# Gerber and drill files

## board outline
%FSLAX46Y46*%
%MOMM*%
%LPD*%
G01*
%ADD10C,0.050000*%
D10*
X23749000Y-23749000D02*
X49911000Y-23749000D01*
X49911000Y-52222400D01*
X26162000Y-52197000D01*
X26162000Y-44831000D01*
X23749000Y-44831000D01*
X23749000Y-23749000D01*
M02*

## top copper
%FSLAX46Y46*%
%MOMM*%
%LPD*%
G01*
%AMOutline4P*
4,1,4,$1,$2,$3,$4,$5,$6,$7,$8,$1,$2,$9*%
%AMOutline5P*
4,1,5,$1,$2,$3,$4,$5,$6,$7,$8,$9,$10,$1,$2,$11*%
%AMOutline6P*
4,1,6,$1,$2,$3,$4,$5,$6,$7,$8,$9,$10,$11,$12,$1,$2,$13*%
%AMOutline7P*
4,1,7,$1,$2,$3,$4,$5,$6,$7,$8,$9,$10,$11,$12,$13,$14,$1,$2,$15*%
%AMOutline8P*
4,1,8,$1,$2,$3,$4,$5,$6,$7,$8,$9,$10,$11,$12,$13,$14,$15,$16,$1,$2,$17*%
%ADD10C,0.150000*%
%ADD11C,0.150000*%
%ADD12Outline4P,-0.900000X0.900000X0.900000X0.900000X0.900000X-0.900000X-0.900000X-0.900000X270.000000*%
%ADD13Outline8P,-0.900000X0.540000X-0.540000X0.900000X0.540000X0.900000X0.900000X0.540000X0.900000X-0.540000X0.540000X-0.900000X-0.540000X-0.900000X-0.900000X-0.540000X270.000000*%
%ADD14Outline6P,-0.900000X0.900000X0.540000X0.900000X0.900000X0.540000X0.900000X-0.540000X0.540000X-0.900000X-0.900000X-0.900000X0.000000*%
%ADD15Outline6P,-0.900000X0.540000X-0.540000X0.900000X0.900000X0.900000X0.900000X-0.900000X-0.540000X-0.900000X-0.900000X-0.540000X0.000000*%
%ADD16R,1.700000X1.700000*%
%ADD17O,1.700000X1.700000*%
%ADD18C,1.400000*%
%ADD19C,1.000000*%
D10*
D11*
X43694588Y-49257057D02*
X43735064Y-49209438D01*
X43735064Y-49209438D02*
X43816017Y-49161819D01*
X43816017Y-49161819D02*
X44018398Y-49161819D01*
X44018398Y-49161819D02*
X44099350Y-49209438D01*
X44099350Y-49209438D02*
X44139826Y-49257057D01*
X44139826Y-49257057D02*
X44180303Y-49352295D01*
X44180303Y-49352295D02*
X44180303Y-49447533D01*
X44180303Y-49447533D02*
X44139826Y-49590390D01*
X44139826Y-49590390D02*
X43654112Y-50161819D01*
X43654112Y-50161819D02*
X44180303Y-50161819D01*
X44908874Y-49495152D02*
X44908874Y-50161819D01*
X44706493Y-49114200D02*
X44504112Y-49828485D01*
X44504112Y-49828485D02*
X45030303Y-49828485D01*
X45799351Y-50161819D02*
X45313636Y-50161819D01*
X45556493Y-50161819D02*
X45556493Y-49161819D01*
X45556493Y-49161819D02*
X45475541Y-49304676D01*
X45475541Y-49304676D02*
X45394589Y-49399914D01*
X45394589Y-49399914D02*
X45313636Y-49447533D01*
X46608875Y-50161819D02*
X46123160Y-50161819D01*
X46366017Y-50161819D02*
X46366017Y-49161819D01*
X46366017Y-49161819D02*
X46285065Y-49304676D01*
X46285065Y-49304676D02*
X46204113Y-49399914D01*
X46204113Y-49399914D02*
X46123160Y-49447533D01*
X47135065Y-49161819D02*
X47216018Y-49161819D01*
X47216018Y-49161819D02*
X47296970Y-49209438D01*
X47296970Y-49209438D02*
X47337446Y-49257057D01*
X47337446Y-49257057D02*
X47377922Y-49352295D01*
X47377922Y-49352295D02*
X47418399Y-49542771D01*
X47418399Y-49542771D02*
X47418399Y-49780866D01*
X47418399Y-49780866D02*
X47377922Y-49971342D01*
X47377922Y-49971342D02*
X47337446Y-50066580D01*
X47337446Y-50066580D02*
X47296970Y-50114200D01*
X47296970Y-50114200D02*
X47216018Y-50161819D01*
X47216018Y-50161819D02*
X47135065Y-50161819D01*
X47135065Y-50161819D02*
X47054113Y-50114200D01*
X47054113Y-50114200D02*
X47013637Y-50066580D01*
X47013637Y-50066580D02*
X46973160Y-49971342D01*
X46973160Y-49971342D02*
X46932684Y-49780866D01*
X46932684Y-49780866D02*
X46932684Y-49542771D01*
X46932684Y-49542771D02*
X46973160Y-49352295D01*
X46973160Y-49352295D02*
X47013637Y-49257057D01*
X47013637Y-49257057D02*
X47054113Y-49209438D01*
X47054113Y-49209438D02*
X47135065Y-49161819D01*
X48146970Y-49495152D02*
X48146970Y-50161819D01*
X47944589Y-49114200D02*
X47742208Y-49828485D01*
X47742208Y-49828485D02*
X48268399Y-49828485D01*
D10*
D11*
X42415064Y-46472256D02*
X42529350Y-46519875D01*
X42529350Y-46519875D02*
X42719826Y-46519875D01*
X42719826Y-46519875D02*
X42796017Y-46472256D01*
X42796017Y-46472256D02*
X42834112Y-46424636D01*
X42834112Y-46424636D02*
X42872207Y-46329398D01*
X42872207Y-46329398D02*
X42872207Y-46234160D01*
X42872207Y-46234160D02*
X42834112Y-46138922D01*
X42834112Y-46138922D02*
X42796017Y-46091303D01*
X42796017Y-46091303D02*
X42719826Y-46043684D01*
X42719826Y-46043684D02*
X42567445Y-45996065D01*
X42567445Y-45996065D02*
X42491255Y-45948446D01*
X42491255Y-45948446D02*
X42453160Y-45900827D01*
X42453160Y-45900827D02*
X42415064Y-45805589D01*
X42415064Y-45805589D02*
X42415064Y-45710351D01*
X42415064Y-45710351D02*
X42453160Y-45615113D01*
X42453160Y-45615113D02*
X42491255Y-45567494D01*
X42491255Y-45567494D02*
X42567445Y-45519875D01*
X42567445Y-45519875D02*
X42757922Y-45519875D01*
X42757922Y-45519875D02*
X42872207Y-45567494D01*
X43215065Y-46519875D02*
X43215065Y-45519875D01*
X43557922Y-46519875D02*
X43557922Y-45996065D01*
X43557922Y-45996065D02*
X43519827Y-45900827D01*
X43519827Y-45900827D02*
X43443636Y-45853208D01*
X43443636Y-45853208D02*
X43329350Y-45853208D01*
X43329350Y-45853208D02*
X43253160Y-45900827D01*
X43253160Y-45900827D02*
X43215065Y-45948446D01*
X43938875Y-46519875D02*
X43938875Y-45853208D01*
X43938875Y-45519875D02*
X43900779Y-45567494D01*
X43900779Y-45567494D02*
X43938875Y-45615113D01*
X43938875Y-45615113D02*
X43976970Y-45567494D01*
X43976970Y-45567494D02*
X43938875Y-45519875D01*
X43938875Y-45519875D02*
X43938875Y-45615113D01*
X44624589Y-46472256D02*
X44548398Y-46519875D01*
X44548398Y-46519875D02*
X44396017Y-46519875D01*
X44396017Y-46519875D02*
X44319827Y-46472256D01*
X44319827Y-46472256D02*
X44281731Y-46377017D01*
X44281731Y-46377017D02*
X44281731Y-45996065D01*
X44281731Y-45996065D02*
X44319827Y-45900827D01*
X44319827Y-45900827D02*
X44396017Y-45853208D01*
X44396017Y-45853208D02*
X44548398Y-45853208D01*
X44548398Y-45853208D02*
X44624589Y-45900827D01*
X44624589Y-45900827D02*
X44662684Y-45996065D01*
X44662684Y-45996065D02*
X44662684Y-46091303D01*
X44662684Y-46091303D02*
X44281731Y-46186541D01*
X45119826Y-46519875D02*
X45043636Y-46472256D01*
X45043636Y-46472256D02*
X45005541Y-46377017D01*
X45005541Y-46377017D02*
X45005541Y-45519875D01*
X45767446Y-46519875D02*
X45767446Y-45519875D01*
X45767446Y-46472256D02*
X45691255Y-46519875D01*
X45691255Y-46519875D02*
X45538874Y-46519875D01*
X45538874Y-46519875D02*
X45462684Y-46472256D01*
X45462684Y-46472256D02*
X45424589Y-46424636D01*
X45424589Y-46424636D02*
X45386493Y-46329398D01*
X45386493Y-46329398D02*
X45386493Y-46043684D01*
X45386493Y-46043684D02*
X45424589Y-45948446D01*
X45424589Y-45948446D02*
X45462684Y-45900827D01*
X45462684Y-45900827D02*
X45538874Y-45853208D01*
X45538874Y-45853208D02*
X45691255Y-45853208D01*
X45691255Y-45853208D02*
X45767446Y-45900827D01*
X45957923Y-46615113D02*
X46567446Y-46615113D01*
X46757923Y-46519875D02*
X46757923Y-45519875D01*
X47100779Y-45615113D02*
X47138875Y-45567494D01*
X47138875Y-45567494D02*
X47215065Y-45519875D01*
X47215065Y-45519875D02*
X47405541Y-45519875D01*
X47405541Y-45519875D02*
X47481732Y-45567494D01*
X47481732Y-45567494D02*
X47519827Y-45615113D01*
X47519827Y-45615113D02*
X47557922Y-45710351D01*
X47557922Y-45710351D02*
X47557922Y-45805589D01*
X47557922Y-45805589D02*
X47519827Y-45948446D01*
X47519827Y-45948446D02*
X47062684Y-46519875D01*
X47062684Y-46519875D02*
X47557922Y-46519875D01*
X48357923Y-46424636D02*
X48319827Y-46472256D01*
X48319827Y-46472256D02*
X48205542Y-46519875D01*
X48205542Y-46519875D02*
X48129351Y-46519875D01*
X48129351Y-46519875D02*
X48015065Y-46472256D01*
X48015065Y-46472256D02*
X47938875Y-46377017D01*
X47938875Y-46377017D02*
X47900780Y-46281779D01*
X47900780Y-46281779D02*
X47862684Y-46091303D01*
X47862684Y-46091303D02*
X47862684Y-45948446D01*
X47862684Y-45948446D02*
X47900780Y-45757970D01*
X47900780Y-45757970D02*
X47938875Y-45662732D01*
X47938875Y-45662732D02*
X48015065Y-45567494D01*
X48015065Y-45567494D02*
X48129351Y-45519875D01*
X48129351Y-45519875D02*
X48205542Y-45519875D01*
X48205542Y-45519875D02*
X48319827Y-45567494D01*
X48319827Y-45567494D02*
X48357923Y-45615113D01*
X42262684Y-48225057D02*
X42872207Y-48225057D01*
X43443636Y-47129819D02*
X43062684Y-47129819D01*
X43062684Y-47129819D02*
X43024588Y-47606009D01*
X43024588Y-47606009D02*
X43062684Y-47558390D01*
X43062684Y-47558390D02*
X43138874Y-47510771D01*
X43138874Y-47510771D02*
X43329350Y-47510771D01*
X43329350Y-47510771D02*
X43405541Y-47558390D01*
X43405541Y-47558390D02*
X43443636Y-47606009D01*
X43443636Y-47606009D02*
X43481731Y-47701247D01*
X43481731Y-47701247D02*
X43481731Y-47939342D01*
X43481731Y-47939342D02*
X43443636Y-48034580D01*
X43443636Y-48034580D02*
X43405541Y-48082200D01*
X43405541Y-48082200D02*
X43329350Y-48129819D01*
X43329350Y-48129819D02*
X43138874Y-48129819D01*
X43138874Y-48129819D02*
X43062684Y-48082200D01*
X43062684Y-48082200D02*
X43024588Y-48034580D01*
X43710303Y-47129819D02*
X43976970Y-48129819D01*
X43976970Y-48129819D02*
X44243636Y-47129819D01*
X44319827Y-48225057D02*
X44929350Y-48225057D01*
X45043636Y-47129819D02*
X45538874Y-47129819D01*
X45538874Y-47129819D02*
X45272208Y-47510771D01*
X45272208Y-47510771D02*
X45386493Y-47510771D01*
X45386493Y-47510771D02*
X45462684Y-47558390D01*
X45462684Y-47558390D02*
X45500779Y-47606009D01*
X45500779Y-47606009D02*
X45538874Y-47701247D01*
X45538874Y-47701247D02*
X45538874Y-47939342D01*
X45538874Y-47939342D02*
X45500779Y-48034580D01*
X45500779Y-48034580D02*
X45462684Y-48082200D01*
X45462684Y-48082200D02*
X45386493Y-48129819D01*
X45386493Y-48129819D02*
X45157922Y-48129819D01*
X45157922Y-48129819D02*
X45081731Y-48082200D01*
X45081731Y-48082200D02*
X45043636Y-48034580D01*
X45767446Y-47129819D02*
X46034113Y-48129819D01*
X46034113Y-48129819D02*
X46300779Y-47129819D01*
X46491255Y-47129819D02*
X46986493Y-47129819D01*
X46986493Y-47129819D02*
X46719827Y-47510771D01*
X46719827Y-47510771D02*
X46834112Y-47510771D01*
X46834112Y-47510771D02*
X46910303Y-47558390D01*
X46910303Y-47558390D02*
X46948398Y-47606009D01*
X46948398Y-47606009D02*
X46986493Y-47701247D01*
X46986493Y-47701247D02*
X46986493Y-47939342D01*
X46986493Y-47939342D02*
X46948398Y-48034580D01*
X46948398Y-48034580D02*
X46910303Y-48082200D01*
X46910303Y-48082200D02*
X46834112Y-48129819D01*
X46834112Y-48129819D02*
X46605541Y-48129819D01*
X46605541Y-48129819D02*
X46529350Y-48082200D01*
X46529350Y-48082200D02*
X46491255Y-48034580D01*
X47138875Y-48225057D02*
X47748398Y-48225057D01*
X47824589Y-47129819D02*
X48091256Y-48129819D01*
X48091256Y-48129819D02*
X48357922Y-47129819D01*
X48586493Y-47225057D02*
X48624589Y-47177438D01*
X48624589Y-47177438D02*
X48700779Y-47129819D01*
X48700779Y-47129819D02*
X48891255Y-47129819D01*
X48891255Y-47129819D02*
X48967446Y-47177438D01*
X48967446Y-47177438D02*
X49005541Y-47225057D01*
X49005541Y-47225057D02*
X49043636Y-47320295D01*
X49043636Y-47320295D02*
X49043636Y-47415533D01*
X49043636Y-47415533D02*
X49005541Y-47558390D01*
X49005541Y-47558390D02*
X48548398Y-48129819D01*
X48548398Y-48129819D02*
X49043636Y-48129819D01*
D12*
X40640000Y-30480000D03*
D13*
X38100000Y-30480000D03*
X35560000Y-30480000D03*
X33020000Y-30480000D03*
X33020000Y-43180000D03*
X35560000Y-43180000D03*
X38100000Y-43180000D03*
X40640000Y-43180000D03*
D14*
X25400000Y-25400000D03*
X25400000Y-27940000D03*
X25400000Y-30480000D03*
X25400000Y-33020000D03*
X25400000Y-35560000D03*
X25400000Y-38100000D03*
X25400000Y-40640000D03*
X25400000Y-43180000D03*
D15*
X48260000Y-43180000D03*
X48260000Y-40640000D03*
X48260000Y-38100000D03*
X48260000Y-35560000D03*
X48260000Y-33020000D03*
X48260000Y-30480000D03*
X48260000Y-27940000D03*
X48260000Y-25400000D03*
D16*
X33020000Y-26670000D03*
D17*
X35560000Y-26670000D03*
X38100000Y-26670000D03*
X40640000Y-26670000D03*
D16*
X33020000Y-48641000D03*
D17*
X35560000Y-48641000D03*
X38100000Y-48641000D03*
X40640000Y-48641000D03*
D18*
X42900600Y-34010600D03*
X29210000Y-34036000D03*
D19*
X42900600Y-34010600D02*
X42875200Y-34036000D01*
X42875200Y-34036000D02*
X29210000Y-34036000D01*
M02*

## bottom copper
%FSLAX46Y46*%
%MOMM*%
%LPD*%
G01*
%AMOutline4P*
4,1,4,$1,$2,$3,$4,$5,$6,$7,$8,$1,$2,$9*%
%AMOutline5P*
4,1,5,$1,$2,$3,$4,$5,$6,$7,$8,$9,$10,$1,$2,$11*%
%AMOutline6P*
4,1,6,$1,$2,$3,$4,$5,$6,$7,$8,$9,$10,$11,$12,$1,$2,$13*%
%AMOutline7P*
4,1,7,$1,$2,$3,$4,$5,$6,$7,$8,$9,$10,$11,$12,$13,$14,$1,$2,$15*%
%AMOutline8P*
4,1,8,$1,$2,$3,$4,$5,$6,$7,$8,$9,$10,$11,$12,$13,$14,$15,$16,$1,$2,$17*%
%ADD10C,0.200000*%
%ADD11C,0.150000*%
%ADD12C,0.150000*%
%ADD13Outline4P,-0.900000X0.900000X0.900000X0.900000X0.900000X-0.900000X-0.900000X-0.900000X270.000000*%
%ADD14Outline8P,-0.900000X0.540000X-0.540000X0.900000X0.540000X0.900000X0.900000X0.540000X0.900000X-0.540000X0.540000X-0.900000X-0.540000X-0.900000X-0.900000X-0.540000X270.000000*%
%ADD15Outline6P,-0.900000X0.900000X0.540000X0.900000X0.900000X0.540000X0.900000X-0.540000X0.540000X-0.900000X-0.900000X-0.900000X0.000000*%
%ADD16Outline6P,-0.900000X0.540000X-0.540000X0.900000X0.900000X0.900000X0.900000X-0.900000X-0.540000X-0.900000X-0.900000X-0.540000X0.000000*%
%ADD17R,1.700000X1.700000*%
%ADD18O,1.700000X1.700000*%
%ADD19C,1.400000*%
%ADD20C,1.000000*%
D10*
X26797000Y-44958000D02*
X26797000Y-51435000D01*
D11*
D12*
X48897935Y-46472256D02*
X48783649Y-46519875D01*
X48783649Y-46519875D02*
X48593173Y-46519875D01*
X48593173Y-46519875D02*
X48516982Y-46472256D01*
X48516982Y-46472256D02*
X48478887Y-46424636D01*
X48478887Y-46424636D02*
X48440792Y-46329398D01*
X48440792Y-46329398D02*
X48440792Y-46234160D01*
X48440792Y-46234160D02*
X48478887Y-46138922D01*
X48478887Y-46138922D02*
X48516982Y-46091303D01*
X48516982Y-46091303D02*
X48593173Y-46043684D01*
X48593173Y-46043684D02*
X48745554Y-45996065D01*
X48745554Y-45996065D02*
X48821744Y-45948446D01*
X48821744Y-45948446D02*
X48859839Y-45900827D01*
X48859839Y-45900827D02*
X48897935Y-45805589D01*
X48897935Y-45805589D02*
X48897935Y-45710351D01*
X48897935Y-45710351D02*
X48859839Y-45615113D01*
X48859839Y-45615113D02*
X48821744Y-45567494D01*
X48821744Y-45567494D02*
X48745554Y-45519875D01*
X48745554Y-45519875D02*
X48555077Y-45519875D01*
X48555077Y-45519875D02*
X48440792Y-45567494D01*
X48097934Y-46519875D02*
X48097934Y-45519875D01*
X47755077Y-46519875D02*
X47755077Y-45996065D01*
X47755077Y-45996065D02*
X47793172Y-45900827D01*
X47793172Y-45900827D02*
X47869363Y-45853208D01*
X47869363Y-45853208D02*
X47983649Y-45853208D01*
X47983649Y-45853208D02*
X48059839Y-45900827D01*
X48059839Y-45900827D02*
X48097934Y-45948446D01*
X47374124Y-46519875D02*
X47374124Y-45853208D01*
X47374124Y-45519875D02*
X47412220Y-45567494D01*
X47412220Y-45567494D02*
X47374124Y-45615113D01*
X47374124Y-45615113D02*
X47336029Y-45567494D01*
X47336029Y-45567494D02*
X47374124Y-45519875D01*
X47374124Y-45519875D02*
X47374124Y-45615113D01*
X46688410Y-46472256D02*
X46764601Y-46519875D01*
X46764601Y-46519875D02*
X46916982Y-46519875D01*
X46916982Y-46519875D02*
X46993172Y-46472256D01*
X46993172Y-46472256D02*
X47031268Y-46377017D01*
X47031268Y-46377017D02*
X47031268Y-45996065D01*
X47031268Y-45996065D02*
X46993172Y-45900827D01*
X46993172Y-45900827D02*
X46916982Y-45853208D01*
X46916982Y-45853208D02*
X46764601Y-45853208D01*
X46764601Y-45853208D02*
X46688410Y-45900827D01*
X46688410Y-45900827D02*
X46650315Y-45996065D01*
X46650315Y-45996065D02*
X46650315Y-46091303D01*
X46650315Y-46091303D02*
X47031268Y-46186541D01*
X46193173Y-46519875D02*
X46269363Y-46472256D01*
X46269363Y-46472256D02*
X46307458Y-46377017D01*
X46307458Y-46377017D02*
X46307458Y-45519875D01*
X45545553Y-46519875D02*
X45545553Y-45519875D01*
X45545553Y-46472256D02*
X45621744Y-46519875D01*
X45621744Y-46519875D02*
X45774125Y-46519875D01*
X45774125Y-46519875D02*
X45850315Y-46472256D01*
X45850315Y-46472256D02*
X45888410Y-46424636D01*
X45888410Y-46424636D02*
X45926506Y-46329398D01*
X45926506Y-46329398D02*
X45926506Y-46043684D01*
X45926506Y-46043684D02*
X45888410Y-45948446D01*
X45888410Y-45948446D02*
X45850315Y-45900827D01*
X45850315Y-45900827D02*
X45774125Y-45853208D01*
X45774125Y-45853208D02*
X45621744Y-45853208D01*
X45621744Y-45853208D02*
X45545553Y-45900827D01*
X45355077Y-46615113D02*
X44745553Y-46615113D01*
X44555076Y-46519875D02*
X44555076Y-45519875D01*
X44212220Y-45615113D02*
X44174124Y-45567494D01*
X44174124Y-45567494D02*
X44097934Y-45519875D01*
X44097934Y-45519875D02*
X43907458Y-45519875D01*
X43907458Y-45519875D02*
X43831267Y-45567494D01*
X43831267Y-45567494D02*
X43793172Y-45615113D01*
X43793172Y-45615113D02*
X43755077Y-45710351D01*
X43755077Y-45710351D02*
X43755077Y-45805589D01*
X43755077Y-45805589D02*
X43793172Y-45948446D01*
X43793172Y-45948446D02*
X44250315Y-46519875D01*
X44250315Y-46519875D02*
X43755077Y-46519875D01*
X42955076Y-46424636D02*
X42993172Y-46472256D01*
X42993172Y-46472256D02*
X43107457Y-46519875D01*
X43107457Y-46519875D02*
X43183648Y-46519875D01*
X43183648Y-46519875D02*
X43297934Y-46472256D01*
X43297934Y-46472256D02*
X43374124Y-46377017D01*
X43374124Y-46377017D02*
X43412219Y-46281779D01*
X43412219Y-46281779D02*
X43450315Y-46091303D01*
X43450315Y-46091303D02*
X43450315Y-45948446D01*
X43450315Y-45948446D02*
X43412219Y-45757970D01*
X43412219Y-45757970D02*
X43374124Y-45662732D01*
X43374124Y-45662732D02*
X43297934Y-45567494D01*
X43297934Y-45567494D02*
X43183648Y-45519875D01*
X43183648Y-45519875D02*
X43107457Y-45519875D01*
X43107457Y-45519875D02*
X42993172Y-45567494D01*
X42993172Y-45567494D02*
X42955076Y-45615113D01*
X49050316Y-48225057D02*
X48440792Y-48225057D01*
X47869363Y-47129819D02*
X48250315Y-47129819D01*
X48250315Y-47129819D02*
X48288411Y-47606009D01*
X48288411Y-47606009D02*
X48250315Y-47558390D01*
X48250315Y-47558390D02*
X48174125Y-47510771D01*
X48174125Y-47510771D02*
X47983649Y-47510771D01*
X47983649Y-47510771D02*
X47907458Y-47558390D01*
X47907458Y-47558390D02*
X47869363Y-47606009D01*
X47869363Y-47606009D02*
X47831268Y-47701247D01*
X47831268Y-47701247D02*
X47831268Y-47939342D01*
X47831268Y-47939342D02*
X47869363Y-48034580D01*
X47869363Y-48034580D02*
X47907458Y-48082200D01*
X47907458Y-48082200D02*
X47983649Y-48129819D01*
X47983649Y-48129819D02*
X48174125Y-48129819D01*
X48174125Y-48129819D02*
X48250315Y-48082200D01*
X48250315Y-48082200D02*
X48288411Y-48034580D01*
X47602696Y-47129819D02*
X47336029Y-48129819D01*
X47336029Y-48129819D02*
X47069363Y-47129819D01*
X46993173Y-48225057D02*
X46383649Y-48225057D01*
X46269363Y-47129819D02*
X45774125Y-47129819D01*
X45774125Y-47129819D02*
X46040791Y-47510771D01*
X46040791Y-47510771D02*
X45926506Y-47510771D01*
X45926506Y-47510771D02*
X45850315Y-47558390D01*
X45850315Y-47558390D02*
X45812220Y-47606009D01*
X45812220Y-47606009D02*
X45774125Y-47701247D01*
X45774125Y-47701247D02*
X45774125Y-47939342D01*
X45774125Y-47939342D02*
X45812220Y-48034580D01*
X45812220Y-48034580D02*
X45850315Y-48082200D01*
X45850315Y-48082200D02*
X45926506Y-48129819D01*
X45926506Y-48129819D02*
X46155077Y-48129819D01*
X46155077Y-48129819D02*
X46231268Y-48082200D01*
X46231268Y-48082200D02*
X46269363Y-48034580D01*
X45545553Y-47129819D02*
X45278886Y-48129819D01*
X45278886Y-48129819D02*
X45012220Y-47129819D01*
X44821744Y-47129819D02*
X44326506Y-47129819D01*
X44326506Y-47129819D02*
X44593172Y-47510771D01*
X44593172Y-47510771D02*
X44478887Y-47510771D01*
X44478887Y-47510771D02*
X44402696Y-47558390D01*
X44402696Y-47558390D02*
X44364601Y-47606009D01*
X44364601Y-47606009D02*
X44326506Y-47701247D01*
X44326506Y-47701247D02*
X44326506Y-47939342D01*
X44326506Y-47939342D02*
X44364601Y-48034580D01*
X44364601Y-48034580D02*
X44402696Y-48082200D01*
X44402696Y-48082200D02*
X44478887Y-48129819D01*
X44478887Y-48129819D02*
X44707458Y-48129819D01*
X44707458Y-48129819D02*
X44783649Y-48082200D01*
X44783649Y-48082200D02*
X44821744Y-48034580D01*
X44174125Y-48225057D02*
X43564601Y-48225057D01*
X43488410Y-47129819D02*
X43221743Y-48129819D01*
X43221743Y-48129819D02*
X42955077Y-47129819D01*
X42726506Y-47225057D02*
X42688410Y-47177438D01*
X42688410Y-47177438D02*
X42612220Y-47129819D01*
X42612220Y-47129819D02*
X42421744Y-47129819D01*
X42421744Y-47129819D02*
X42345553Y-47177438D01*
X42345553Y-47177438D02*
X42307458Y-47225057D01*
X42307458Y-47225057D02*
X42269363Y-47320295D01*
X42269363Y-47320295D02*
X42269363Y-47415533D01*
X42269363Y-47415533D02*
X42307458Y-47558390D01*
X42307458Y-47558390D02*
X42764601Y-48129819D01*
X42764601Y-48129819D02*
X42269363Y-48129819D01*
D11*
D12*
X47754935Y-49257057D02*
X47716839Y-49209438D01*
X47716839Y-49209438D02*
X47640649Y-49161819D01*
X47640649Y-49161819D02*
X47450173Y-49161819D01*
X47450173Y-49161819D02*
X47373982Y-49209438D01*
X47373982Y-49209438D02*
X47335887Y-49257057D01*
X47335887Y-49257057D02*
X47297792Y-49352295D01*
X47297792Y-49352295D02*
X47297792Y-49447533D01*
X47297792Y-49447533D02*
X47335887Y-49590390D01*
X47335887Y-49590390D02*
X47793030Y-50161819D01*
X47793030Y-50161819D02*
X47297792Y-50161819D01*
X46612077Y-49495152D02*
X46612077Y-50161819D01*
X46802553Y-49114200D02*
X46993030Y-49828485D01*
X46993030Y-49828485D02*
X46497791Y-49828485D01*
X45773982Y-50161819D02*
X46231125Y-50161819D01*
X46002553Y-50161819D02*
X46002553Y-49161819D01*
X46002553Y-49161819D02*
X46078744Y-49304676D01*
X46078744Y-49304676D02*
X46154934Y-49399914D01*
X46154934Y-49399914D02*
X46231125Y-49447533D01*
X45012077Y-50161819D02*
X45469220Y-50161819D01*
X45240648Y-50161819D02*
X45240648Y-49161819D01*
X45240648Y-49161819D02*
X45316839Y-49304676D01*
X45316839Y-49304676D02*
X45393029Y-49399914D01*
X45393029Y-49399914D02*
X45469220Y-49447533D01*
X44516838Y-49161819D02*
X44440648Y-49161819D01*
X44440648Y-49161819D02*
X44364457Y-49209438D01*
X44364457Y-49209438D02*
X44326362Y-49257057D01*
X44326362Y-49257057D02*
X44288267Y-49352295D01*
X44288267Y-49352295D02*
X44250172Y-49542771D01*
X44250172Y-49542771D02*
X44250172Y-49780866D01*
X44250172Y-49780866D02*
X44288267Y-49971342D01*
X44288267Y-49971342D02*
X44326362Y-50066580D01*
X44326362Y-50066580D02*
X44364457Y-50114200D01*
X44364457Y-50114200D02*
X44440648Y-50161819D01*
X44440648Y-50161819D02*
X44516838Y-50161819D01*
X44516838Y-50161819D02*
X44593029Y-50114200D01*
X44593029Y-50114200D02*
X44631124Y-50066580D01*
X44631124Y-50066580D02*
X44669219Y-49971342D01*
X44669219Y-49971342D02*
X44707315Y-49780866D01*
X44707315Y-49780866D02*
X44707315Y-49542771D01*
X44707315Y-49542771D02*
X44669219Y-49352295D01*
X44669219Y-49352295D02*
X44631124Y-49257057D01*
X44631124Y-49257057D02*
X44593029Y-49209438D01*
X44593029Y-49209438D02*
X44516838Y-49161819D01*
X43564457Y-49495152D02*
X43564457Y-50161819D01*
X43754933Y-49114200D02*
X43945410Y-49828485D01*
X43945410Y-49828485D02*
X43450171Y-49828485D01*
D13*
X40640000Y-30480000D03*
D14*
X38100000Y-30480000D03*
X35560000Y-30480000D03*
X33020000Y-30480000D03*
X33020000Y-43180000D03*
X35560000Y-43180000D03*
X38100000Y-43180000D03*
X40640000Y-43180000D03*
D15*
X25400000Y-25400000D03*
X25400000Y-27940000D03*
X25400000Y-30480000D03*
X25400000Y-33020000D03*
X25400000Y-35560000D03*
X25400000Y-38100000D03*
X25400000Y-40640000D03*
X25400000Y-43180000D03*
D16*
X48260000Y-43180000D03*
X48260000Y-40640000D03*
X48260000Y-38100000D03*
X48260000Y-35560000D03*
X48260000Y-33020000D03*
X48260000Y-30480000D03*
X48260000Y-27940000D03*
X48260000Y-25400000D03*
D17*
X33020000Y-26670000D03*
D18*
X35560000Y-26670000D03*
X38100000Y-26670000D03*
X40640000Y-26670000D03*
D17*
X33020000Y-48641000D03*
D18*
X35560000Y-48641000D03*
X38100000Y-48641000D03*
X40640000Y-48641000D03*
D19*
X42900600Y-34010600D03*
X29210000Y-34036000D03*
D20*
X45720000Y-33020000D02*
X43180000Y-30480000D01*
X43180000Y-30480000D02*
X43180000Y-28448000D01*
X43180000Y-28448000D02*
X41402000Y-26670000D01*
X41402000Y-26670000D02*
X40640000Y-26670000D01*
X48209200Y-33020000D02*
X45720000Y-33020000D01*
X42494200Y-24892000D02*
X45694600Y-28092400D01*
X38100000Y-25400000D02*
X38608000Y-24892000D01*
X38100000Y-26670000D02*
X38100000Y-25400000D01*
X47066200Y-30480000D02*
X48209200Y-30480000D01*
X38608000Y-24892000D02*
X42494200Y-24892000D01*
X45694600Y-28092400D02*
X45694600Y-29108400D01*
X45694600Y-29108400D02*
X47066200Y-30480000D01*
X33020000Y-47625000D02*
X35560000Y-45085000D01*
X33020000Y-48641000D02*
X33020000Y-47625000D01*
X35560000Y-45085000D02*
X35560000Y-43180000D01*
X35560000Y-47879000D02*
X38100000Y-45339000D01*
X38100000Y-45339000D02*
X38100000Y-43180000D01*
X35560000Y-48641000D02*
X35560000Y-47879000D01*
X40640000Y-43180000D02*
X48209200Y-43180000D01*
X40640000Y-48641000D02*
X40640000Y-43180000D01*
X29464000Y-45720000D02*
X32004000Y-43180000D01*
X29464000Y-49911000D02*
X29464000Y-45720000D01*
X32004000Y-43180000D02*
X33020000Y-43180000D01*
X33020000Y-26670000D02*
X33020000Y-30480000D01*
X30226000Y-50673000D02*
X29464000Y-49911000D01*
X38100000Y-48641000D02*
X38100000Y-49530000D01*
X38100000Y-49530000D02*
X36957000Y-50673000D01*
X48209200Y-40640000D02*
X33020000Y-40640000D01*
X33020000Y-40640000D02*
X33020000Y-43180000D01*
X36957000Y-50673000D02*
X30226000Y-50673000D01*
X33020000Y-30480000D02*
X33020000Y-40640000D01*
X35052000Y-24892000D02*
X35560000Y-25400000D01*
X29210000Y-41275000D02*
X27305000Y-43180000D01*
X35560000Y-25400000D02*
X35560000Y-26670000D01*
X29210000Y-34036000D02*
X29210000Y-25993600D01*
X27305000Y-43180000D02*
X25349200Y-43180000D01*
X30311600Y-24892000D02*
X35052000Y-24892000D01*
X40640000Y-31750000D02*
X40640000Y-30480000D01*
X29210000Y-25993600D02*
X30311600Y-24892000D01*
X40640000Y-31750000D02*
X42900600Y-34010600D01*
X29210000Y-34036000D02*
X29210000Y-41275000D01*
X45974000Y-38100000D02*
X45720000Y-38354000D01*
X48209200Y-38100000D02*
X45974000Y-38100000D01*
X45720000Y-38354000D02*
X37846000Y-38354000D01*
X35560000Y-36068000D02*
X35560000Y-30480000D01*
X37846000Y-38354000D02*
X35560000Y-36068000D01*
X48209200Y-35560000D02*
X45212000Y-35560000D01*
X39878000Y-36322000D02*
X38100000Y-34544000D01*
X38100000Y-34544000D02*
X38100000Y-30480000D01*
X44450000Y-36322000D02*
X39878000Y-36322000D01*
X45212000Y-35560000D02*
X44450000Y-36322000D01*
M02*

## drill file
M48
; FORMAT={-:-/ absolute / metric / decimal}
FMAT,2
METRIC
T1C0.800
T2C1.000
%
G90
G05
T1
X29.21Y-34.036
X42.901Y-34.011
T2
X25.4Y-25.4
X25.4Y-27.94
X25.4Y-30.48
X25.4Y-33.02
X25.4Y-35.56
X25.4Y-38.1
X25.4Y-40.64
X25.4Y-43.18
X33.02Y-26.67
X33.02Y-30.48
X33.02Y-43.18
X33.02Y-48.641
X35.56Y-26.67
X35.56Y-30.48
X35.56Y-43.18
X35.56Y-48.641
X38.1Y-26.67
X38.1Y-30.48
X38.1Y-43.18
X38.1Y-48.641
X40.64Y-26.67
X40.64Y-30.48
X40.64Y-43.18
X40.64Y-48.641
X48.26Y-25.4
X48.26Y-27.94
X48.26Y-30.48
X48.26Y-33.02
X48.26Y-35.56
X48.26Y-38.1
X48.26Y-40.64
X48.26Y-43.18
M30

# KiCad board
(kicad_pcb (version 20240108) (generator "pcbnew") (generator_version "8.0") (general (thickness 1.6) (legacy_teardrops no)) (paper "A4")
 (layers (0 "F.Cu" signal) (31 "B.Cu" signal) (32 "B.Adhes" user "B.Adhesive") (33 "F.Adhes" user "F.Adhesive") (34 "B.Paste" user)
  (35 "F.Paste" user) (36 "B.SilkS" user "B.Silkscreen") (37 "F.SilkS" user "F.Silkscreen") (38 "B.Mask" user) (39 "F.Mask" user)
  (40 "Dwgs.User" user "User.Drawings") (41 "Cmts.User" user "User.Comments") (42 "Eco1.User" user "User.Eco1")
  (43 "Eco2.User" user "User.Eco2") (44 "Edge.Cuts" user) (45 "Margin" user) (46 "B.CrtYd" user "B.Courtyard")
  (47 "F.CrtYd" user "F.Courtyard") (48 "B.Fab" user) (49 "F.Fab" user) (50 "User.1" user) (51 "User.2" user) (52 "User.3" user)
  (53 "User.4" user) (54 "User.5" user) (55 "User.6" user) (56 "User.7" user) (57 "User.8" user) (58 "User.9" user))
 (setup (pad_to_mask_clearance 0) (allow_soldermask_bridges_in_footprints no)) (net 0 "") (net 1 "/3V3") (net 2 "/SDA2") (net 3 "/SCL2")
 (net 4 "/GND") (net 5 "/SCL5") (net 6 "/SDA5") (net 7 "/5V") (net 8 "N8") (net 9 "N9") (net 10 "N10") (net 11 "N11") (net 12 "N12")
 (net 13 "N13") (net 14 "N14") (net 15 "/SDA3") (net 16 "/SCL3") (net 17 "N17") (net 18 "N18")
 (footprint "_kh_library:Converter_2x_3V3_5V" (layer "F.Cu") (at 40.64 30.48 -90)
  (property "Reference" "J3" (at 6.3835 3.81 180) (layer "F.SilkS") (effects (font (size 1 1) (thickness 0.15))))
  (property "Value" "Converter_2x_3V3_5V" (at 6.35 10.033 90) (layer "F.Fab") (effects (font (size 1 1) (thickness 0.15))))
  (pad "1" thru_hole roundrect (at 0 0 270) (size 1.8 1.8) (drill 1) (layers "*.Cu" "*.Mask") (remove_unused_layers no) (roundrect_rratio 0)
   (chamfer_ratio 0.2) (chamfer) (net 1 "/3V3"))
  (pad "2" thru_hole roundrect (at 0 2.54 270) (size 1.8 1.8) (drill 1) (layers "*.Cu" "*.Mask") (remove_unused_layers no)
   (roundrect_rratio 0) (chamfer_ratio 0.2) (chamfer top_left top_right bottom_left bottom_right) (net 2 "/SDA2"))
  (pad "3" thru_hole roundrect (at 0 5.08 270) (size 1.8 1.8) (drill 1) (layers "*.Cu" "*.Mask") (remove_unused_layers no)
   (roundrect_rratio 0) (chamfer_ratio 0.2) (chamfer top_left top_right bottom_left bottom_right) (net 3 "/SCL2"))
  (pad "4" thru_hole roundrect (at 0 7.62 270) (size 1.8 1.8) (drill 1) (layers "*.Cu" "*.Mask") (remove_unused_layers no)
   (roundrect_rratio 0) (chamfer_ratio 0.2) (chamfer top_left top_right bottom_left bottom_right) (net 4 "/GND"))
  (pad "5" thru_hole roundrect (at 12.7 7.62 270) (size 1.8 1.8) (drill 1) (layers "*.Cu" "*.Mask") (remove_unused_layers no)
   (roundrect_rratio 0) (chamfer_ratio 0.2) (chamfer top_left top_right bottom_left bottom_right) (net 4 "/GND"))
  (pad "6" thru_hole roundrect (at 12.7 5.08 270) (size 1.8 1.8) (drill 1) (layers "*.Cu" "*.Mask") (remove_unused_layers no)
   (roundrect_rratio 0) (chamfer_ratio 0.2) (chamfer top_left top_right bottom_left bottom_right) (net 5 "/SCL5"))
  (pad "7" thru_hole roundrect (at 12.7 2.54 270) (size 1.8 1.8) (drill 1) (layers "*.Cu" "*.Mask") (remove_unused_layers no)
   (roundrect_rratio 0) (chamfer_ratio 0.2) (chamfer top_left top_right bottom_left bottom_right) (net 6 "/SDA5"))
  (pad "8" thru_hole roundrect (at 12.7 0 270) (size 1.8 1.8) (drill 1) (layers "*.Cu" "*.Mask") (remove_unused_layers no)
   (roundrect_rratio 0) (chamfer_ratio 0.2) (chamfer top_left top_right bottom_left bottom_right) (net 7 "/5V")))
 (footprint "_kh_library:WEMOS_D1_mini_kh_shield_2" (layer "F.Cu") (at 25.4 25.4)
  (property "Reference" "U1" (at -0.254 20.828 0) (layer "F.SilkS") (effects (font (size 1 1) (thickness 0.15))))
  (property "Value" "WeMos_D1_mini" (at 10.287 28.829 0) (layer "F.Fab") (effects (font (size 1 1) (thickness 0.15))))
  (pad "1" thru_hole roundrect (at 0 0) (size 1.8 1.8) (drill 1) (layers "*.Cu" "*.Mask") (remove_unused_layers no) (roundrect_rratio 0)
   (chamfer_ratio 0.2) (chamfer top_right bottom_right) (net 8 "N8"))
  (pad "2" thru_hole roundrect (at 0 2.54) (size 1.8 1.8) (drill 1) (layers "*.Cu" "*.Mask") (remove_unused_layers no) (roundrect_rratio 0)
   (chamfer_ratio 0.2) (chamfer top_right bottom_right) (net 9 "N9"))
  (pad "3" thru_hole roundrect (at 0 5.08) (size 1.8 1.8) (drill 1) (layers "*.Cu" "*.Mask") (remove_unused_layers no) (roundrect_rratio 0)
   (chamfer_ratio 0.2) (chamfer top_right bottom_right) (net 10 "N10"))
  (pad "4" thru_hole roundrect (at 0 7.62) (size 1.8 1.8) (drill 1) (layers "*.Cu" "*.Mask") (remove_unused_layers no) (roundrect_rratio 0)
   (chamfer_ratio 0.2) (chamfer top_right bottom_right) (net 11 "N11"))
  (pad "5" thru_hole roundrect (at 0 10.16) (size 1.8 1.8) (drill 1) (layers "*.Cu" "*.Mask") (remove_unused_layers no) (roundrect_rratio 0)
   (chamfer_ratio 0.2) (chamfer top_right bottom_right) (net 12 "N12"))
  (pad "6" thru_hole roundrect (at 0 12.7) (size 1.8 1.8) (drill 1) (layers "*.Cu" "*.Mask") (remove_unused_layers no) (roundrect_rratio 0)
   (chamfer_ratio 0.2) (chamfer top_right bottom_right) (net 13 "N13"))
  (pad "7" thru_hole roundrect (at 0 15.24) (size 1.8 1.8) (drill 1) (layers "*.Cu" "*.Mask") (remove_unused_layers no) (roundrect_rratio 0)
   (chamfer_ratio 0.2) (chamfer top_right bottom_right) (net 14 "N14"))
  (pad "8" thru_hole roundrect (at 0 17.78) (size 1.8 1.8) (drill 1) (layers "*.Cu" "*.Mask") (remove_unused_layers no) (roundrect_rratio 0)
   (chamfer_ratio 0.2) (chamfer top_right bottom_right) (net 1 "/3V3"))
  (pad "9" thru_hole roundrect (at 22.86 17.78) (size 1.8 1.8) (drill 1) (layers "*.Cu" "*.Mask") (remove_unused_layers no)
   (roundrect_rratio 0) (chamfer_ratio 0.2) (chamfer top_left bottom_left) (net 7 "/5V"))
  (pad "10" thru_hole roundrect (at 22.86 15.24) (size 1.8 1.8) (drill 1) (layers "*.Cu" "*.Mask") (remove_unused_layers no)
   (roundrect_rratio 0) (chamfer_ratio 0.2) (chamfer top_left bottom_left) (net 4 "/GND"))
  (pad "11" thru_hole roundrect (at 22.86 12.7) (size 1.8 1.8) (drill 1) (layers "*.Cu" "*.Mask") (remove_unused_layers no)
   (roundrect_rratio 0) (chamfer_ratio 0.2) (chamfer top_left bottom_left) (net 3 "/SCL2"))
  (pad "12" thru_hole roundrect (at 22.86 10.16) (size 1.8 1.8) (drill 1) (layers "*.Cu" "*.Mask") (remove_unused_layers no)
   (roundrect_rratio 0) (chamfer_ratio 0.2) (chamfer top_left bottom_left) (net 2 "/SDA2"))
  (pad "13" thru_hole roundrect (at 22.86 7.62) (size 1.8 1.8) (drill 1) (layers "*.Cu" "*.Mask") (remove_unused_layers no)
   (roundrect_rratio 0) (chamfer_ratio 0.2) (chamfer top_left bottom_left) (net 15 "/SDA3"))
  (pad "14" thru_hole roundrect (at 22.86 5.08) (size 1.8 1.8) (drill 1) (layers "*.Cu" "*.Mask") (remove_unused_layers no)
   (roundrect_rratio 0) (chamfer_ratio 0.2) (chamfer top_left bottom_left) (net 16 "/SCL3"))
  (pad "15" thru_hole roundrect (at 22.86 2.54) (size 1.8 1.8) (drill 1) (layers "*.Cu" "*.Mask") (remove_unused_layers no)
   (roundrect_rratio 0) (chamfer_ratio 0.2) (chamfer top_left bottom_left) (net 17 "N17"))
  (pad "16" thru_hole roundrect (at 22.86 0) (size 1.8 1.8) (drill 1) (layers "*.Cu" "*.Mask") (remove_unused_layers no)
   (roundrect_rratio 0) (chamfer_ratio 0.2) (chamfer top_left bottom_left) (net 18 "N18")))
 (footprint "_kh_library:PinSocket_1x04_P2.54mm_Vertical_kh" (layer "F.Cu") (at 33.02 26.67 90)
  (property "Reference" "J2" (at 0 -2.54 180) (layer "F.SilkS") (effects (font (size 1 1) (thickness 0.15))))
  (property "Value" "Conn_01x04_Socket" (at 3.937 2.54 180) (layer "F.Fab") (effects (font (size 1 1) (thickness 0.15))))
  (pad "1" thru_hole rect (at 0 0 90) (size 1.7 1.7) (drill 1) (layers "*.Cu" "*.Mask") (remove_unused_layers no) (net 4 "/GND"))
  (pad "2" thru_hole oval (at 0 2.54 90) (size 1.7 1.7) (drill 1) (layers "*.Cu" "*.Mask") (remove_unused_layers no) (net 1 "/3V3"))
  (pad "3" thru_hole oval (at 0 5.08 90) (size 1.7 1.7) (drill 1) (layers "*.Cu" "*.Mask") (remove_unused_layers no) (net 16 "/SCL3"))
  (pad "4" thru_hole oval (at 0 7.62 90) (size 1.7 1.7) (drill 1) (layers "*.Cu" "*.Mask") (remove_unused_layers no) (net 15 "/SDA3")))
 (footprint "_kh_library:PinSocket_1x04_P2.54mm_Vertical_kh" (layer "F.Cu") (at 33.02 48.641 90)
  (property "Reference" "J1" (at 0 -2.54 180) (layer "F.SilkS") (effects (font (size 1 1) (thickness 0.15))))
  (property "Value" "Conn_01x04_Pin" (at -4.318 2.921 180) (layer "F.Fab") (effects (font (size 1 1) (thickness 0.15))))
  (pad "1" thru_hole rect (at 0 0 90) (size 1.7 1.7) (drill 1) (layers "*.Cu" "*.Mask") (remove_unused_layers no) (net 5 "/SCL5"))
  (pad "2" thru_hole oval (at 0 2.54 90) (size 1.7 1.7) (drill 1) (layers "*.Cu" "*.Mask") (remove_unused_layers no) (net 6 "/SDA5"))
  (pad "3" thru_hole oval (at 0 5.08 90) (size 1.7 1.7) (drill 1) (layers "*.Cu" "*.Mask") (remove_unused_layers no) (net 4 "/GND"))
  (pad "4" thru_hole oval (at 0 7.62 90) (size 1.7 1.7) (drill 1) (layers "*.Cu" "*.Mask") (remove_unused_layers no) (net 7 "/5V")))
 (gr_line (start 26.797 44.958) (end 26.797 51.435) (stroke (width 0.2) (type default)) (layer "B.Cu"))
 (gr_poly
  (pts (xy 23.749 23.749) (xy 49.911 23.749) (xy 49.911 52.2224) (xy 26.162 52.197) (xy 26.162 44.831) (xy 23.749 44.831))
  (stroke (width 0.05) (type solid)) (fill none) (layer "Edge.Cuts"))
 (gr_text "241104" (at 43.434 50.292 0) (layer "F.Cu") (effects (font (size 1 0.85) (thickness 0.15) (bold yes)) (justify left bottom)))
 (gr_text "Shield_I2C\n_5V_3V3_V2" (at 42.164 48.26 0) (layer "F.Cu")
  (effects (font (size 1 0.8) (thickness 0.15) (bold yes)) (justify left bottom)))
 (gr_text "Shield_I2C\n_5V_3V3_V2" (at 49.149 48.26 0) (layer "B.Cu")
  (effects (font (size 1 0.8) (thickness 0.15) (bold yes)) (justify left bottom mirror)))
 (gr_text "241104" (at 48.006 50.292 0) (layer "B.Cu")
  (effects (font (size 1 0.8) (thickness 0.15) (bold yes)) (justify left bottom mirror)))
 (segment (start 45.72 33.02) (end 43.18 30.48) (width 1) (layer "B.Cu") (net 15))
 (segment (start 43.18 30.48) (end 43.18 28.448) (width 1) (layer "B.Cu") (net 15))
 (segment (start 43.18 28.448) (end 41.402 26.67) (width 1) (layer "B.Cu") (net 15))
 (segment (start 41.402 26.67) (end 40.64 26.67) (width 1) (layer "B.Cu") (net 15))
 (segment (start 48.2092 33.02) (end 45.72 33.02) (width 1) (layer "B.Cu") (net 15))
 (segment (start 42.4942 24.892) (end 45.6946 28.0924) (width 1) (layer "B.Cu") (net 16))
 (segment (start 38.1 25.4) (end 38.608 24.892) (width 1) (layer "B.Cu") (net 16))
 (segment (start 38.1 26.67) (end 38.1 25.4) (width 1) (layer "B.Cu") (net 16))
 (segment (start 47.0662 30.48) (end 48.2092 30.48) (width 1) (layer "B.Cu") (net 16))
 (segment (start 38.608 24.892) (end 42.4942 24.892) (width 1) (layer "B.Cu") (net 16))
 (segment (start 45.6946 28.0924) (end 45.6946 29.1084) (width 1) (layer "B.Cu") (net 16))
 (segment (start 45.6946 29.1084) (end 47.0662 30.48) (width 1) (layer "B.Cu") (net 16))
 (segment (start 33.02 47.625) (end 35.56 45.085) (width 1) (layer "B.Cu") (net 5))
 (segment (start 33.02 48.641) (end 33.02 47.625) (width 1) (layer "B.Cu") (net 5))
 (segment (start 35.56 45.085) (end 35.56 43.18) (width 1) (layer "B.Cu") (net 5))
 (segment (start 35.56 47.879) (end 38.1 45.339) (width 1) (layer "B.Cu") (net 6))
 (segment (start 38.1 45.339) (end 38.1 43.18) (width 1) (layer "B.Cu") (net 6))
 (segment (start 35.56 48.641) (end 35.56 47.879) (width 1) (layer "B.Cu") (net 6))
 (segment (start 40.64 43.18) (end 48.2092 43.18) (width 1) (layer "B.Cu") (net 7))
 (segment (start 40.64 48.641) (end 40.64 43.18) (width 1) (layer "B.Cu") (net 7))
 (segment (start 29.464 45.72) (end 32.004 43.18) (width 1) (layer "B.Cu") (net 4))
 (segment (start 29.464 49.911) (end 29.464 45.72) (width 1) (layer "B.Cu") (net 4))
 (segment (start 32.004 43.18) (end 33.02 43.18) (width 1) (layer "B.Cu") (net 4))
 (segment (start 33.02 26.67) (end 33.02 30.48) (width 1) (layer "B.Cu") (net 4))
 (segment (start 30.226 50.673) (end 29.464 49.911) (width 1) (layer "B.Cu") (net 4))
 (segment (start 38.1 48.641) (end 38.1 49.53) (width 1) (layer "B.Cu") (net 4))
 (segment (start 38.1 49.53) (end 36.957 50.673) (width 1) (layer "B.Cu") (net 4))
 (segment (start 48.2092 40.64) (end 33.02 40.64) (width 1) (layer "B.Cu") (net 4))
 (segment (start 33.02 40.64) (end 33.02 43.18) (width 1) (layer "B.Cu") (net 4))
 (segment (start 36.957 50.673) (end 30.226 50.673) (width 1) (layer "B.Cu") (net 4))
 (segment (start 33.02 30.48) (end 33.02 40.64) (width 1) (layer "B.Cu") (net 4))
 (segment (start 42.9006 34.0106) (end 42.8752 34.036) (width 1) (layer "F.Cu") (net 1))
 (segment (start 42.8752 34.036) (end 29.21 34.036) (width 1) (layer "F.Cu") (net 1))
 (via (at 42.9006 34.0106) (size 1.4) (drill 0.8) (layers "F.Cu" "B.Cu") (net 1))
 (via (at 29.21 34.036) (size 1.4) (drill 0.8) (layers "F.Cu" "B.Cu") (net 1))
 (segment (start 35.052 24.892) (end 35.56 25.4) (width 1) (layer "B.Cu") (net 1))
 (segment (start 29.21 41.275) (end 27.305 43.18) (width 1) (layer "B.Cu") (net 1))
 (segment (start 35.56 25.4) (end 35.56 26.67) (width 1) (layer "B.Cu") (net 1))
 (segment (start 29.21 34.036) (end 29.21 25.9936) (width 1) (layer "B.Cu") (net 1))
 (segment (start 27.305 43.18) (end 25.3492 43.18) (width 1) (layer "B.Cu") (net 1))
 (segment (start 30.3116 24.892) (end 35.052 24.892) (width 1) (layer "B.Cu") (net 1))
 (segment (start 40.64 31.75) (end 40.64 30.48) (width 1) (layer "B.Cu") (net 1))
 (segment (start 29.21 25.9936) (end 30.3116 24.892) (width 1) (layer "B.Cu") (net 1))
 (segment (start 40.64 31.75) (end 42.9006 34.0106) (width 1) (layer "B.Cu") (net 1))
 (segment (start 29.21 34.036) (end 29.21 41.275) (width 1) (layer "B.Cu") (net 1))
 (segment (start 45.974 38.1) (end 45.72 38.354) (width 1) (layer "B.Cu") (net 3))
 (segment (start 48.2092 38.1) (end 45.974 38.1) (width 1) (layer "B.Cu") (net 3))
 (segment (start 45.72 38.354) (end 37.846 38.354) (width 1) (layer "B.Cu") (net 3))
 (segment (start 35.56 36.068) (end 35.56 30.48) (width 1) (layer "B.Cu") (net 3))
 (segment (start 37.846 38.354) (end 35.56 36.068) (width 1) (layer "B.Cu") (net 3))
 (segment (start 48.2092 35.56) (end 45.212 35.56) (width 1) (layer "B.Cu") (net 2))
 (segment (start 39.878 36.322) (end 38.1 34.544) (width 1) (layer "B.Cu") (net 2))
 (segment (start 38.1 34.544) (end 38.1 30.48) (width 1) (layer "B.Cu") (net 2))
 (segment (start 44.45 36.322) (end 39.878 36.322) (width 1) (layer "B.Cu") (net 2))
 (segment (start 45.212 35.56) (end 44.45 36.322) (width 1) (layer "B.Cu") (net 2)))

